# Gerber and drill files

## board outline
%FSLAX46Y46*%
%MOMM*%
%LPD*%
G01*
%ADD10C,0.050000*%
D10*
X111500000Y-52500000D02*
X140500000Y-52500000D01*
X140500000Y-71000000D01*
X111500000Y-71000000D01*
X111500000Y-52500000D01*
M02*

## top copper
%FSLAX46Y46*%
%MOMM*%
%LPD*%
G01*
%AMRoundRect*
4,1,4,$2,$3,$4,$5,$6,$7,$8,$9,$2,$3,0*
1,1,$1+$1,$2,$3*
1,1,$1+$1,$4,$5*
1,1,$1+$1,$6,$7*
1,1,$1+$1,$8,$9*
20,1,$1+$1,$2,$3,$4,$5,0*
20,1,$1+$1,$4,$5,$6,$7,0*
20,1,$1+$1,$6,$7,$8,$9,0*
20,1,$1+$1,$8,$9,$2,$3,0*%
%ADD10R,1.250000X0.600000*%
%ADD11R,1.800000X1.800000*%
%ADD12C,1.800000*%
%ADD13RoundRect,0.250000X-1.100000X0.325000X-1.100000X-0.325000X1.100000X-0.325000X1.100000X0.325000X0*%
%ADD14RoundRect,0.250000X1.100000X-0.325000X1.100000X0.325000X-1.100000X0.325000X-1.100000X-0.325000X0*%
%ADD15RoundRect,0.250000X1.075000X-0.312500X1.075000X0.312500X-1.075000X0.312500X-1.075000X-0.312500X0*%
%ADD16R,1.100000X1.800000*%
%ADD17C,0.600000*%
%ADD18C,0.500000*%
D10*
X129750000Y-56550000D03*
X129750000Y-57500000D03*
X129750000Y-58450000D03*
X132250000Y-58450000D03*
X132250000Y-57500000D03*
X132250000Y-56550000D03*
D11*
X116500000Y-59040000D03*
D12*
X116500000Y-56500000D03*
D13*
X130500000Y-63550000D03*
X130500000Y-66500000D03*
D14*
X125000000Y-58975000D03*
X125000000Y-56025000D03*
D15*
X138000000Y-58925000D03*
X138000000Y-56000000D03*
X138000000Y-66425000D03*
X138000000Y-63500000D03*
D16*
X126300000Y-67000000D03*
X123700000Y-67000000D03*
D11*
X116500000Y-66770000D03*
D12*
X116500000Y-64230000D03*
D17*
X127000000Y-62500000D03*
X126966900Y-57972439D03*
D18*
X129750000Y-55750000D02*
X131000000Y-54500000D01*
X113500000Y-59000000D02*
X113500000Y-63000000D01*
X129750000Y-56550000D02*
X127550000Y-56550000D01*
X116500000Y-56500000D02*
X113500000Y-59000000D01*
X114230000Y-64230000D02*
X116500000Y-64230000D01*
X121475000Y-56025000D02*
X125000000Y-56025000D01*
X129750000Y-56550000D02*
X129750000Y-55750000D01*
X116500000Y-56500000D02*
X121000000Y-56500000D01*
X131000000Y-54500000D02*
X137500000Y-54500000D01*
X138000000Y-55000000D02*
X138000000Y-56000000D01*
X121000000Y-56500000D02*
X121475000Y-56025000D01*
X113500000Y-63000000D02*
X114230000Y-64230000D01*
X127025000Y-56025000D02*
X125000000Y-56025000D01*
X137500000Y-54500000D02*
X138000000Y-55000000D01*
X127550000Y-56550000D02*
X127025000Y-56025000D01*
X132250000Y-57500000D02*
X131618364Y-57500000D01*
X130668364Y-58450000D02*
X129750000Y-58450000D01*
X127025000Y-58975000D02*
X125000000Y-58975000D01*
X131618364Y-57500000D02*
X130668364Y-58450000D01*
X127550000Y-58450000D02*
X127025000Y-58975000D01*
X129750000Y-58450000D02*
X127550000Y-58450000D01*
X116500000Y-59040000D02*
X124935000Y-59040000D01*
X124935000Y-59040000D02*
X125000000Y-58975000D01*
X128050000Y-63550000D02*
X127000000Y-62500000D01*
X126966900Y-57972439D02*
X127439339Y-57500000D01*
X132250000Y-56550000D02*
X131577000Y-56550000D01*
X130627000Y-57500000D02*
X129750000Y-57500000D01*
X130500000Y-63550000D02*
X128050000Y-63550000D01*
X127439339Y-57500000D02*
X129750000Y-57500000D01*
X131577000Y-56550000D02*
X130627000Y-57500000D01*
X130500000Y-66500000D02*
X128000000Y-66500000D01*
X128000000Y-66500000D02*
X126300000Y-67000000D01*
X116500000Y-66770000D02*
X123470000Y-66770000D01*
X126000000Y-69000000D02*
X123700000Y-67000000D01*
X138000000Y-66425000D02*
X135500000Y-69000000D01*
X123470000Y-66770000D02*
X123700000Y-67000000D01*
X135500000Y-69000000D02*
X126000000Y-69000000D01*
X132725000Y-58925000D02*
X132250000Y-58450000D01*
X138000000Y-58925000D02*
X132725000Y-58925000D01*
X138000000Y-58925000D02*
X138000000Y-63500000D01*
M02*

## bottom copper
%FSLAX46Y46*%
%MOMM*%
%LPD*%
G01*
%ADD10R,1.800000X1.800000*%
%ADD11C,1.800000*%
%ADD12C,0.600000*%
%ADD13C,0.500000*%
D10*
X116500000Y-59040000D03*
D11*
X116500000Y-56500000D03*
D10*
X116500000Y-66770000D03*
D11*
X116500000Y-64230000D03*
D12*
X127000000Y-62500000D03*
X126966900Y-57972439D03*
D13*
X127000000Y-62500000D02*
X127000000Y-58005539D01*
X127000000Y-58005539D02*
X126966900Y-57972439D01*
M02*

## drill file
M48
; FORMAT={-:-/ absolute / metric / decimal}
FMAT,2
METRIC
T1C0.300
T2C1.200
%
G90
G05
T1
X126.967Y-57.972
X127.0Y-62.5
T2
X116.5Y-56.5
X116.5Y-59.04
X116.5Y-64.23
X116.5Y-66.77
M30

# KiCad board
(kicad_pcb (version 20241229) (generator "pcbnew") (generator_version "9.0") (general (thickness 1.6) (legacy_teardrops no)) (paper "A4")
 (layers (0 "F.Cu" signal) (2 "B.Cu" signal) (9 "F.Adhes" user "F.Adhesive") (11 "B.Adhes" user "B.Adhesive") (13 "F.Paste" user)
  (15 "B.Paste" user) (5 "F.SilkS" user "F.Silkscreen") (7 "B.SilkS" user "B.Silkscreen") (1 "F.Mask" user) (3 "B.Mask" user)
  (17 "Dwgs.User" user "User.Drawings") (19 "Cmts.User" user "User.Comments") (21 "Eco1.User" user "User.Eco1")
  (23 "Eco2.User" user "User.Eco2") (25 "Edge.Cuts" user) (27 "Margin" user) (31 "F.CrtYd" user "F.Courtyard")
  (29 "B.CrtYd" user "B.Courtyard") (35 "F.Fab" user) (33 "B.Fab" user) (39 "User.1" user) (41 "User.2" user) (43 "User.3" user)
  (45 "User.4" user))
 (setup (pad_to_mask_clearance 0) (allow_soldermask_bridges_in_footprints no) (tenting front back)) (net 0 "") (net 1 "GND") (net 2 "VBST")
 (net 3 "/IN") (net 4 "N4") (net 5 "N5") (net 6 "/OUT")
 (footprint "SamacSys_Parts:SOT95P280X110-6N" (layer "F.Cu") (at 131 57.5)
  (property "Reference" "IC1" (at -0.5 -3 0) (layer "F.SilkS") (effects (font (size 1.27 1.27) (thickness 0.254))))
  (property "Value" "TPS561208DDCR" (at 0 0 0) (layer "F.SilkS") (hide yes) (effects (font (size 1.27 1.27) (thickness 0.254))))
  (pad "1" smd rect (at -1.25 -0.95 90) (size 0.6 1.25) (layers "F.Cu" "F.Mask" "F.Paste") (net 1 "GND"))
  (pad "2" smd rect (at -1.25 0 90) (size 0.6 1.25) (layers "F.Cu" "F.Mask" "F.Paste") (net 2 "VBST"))
  (pad "3" smd rect (at -1.25 0.95 90) (size 0.6 1.25) (layers "F.Cu" "F.Mask" "F.Paste") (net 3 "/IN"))
  (pad "4" smd rect (at 1.25 0.95 90) (size 0.6 1.25) (layers "F.Cu" "F.Mask" "F.Paste") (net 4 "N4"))
  (pad "5" smd rect (at 1.25 0 90) (size 0.6 1.25) (layers "F.Cu" "F.Mask" "F.Paste") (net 3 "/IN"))
  (pad "6" smd rect (at 1.25 -0.95 90) (size 0.6 1.25) (layers "F.Cu" "F.Mask" "F.Paste") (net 2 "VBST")))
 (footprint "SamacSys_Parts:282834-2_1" (layer "F.Cu") (at 116.5 59.04 90)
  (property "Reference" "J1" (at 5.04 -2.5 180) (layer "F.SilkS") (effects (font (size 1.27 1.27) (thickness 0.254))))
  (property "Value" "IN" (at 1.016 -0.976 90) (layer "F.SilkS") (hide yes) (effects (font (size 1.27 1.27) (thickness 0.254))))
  (pad "1" thru_hole rect (at 0 0 90) (size 1.8 1.8) (drill 1.2) (layers "*.Cu" "*.Mask") (remove_unused_layers no) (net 3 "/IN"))
  (pad "2" thru_hole circle (at 2.54 0 90) (size 1.8 1.8) (drill 1.2) (layers "*.Cu" "*.Mask") (remove_unused_layers no) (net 1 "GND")))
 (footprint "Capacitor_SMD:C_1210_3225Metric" (layer "F.Cu") (at 130.5 65.025 -90)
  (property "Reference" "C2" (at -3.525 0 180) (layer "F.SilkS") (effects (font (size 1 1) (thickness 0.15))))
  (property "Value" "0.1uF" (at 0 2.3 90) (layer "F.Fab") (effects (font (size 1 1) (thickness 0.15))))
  (pad "1" smd roundrect (at -1.475 0 270) (size 1.15 2.7) (layers "F.Cu" "F.Mask" "F.Paste") (roundrect_rratio 0.217391) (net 2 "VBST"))
  (pad "2" smd roundrect (at 1.475 0 270) (size 1.15 2.7) (layers "F.Cu" "F.Mask" "F.Paste") (roundrect_rratio 0.217391) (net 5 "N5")))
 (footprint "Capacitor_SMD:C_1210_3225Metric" (layer "F.Cu") (at 125 57.5 90)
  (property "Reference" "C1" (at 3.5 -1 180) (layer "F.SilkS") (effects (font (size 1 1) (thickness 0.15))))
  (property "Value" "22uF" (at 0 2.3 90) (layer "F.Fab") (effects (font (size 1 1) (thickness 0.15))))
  (pad "1" smd roundrect (at -1.475 0 90) (size 1.15 2.7) (layers "F.Cu" "F.Mask" "F.Paste") (roundrect_rratio 0.217391) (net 3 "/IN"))
  (pad "2" smd roundrect (at 1.475 0 90) (size 1.15 2.7) (layers "F.Cu" "F.Mask" "F.Paste") (roundrect_rratio 0.217391) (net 1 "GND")))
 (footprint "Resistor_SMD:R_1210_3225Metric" (layer "F.Cu") (at 138 57.4625 90)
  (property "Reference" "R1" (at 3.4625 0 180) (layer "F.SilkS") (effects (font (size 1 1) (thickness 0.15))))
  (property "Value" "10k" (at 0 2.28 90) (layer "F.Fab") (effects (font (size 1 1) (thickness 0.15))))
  (pad "1" smd roundrect (at -1.4625 0 90) (size 1.125 2.65) (layers "F.Cu" "F.Mask" "F.Paste") (roundrect_rratio 0.222222) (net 4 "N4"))
  (pad "2" smd roundrect (at 1.4625 0 90) (size 1.125 2.65) (layers "F.Cu" "F.Mask" "F.Paste") (roundrect_rratio 0.222222) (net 1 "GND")))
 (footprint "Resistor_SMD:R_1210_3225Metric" (layer "F.Cu") (at 138 64.9625 90)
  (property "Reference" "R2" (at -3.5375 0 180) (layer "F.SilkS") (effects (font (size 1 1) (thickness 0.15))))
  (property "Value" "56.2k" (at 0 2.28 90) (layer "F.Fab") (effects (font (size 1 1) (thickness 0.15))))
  (pad "1" smd roundrect (at -1.4625 0 90) (size 1.125 2.65) (layers "F.Cu" "F.Mask" "F.Paste") (roundrect_rratio 0.222222) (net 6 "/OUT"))
  (pad "2" smd roundrect (at 1.4625 0 90) (size 1.125 2.65) (layers "F.Cu" "F.Mask" "F.Paste") (roundrect_rratio 0.222222) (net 4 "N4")))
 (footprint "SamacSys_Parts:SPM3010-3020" (layer "F.Cu") (at 125 67 180)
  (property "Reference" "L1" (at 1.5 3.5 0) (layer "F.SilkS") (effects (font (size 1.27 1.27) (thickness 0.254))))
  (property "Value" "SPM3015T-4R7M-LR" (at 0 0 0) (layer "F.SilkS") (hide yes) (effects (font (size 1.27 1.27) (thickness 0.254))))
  (pad "1" smd rect (at -1.3 0 180) (size 1.1 1.8) (layers "F.Cu" "F.Mask" "F.Paste") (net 5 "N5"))
  (pad "2" smd rect (at 1.3 0 180) (size 1.1 1.8) (layers "F.Cu" "F.Mask" "F.Paste") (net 6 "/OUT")))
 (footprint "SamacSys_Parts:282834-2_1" (layer "F.Cu") (at 116.5 66.77 90)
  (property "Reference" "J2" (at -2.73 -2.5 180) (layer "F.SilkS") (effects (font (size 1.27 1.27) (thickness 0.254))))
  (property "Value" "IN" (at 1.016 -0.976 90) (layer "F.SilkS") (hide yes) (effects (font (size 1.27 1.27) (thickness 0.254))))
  (pad "1" thru_hole rect (at 0 0 90) (size 1.8 1.8) (drill 1.2) (layers "*.Cu" "*.Mask") (remove_unused_layers no) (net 6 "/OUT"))
  (pad "2" thru_hole circle (at 2.54 0 90) (size 1.8 1.8) (drill 1.2) (layers "*.Cu" "*.Mask") (remove_unused_layers no) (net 1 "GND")))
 (gr_rect (start 111.5 52.5) (end 140.5 71) (stroke (width 0.05) (type default)) (fill no) (layer "Edge.Cuts"))
 (segment (start 129.75 55.75) (end 131 54.5) (width 0.5) (layer "F.Cu") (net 1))
 (segment (start 113.5 59) (end 113.5 63) (width 0.5) (layer "F.Cu") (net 1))
 (segment (start 129.75 56.55) (end 127.55 56.55) (width 0.5) (layer "F.Cu") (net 1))
 (segment (start 116.5 56.5) (end 113.5 59) (width 0.5) (layer "F.Cu") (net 1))
 (segment (start 114.23 64.23) (end 116.5 64.23) (width 0.5) (layer "F.Cu") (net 1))
 (segment (start 121.475 56.025) (end 125 56.025) (width 0.5) (layer "F.Cu") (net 1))
 (segment (start 129.75 56.55) (end 129.75 55.75) (width 0.5) (layer "F.Cu") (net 1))
 (segment (start 116.5 56.5) (end 121 56.5) (width 0.5) (layer "F.Cu") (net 1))
 (segment (start 131 54.5) (end 137.5 54.5) (width 0.5) (layer "F.Cu") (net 1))
 (segment (start 138 55) (end 138 56) (width 0.5) (layer "F.Cu") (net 1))
 (segment (start 121 56.5) (end 121.475 56.025) (width 0.5) (layer "F.Cu") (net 1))
 (segment (start 113.5 63) (end 114.23 64.23) (width 0.5) (layer "F.Cu") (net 1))
 (segment (start 127.025 56.025) (end 125 56.025) (width 0.5) (layer "F.Cu") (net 1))
 (segment (start 137.5 54.5) (end 138 55) (width 0.5) (layer "F.Cu") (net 1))
 (segment (start 127.55 56.55) (end 127.025 56.025) (width 0.5) (layer "F.Cu") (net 1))
 (segment (start 132.25 57.5) (end 131.618364 57.5) (width 0.5) (layer "F.Cu") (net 3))
 (segment (start 130.668364 58.45) (end 129.75 58.45) (width 0.5) (layer "F.Cu") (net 3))
 (segment (start 127.025 58.975) (end 125 58.975) (width 0.5) (layer "F.Cu") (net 3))
 (segment (start 131.618364 57.5) (end 130.668364 58.45) (width 0.5) (layer "F.Cu") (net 3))
 (segment (start 127.55 58.45) (end 127.025 58.975) (width 0.5) (layer "F.Cu") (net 3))
 (segment (start 129.75 58.45) (end 127.55 58.45) (width 0.5) (layer "F.Cu") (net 3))
 (segment (start 116.5 59.04) (end 124.935 59.04) (width 0.5) (layer "F.Cu") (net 3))
 (segment (start 124.935 59.04) (end 125 58.975) (width 0.5) (layer "F.Cu") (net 3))
 (segment (start 128.05 63.55) (end 127 62.5) (width 0.5) (layer "F.Cu") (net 2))
 (segment (start 126.9669 57.972439) (end 127.439339 57.5) (width 0.5) (layer "F.Cu") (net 2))
 (segment (start 132.25 56.55) (end 131.577 56.55) (width 0.5) (layer "F.Cu") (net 2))
 (segment (start 130.627 57.5) (end 129.75 57.5) (width 0.5) (layer "F.Cu") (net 2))
 (segment (start 130.5 63.55) (end 128.05 63.55) (width 0.5) (layer "F.Cu") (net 2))
 (segment (start 127.439339 57.5) (end 129.75 57.5) (width 0.5) (layer "F.Cu") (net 2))
 (segment (start 131.577 56.55) (end 130.627 57.5) (width 0.5) (layer "F.Cu") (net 2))
 (via (at 127 62.5) (size 0.6) (drill 0.3) (layers "F.Cu" "B.Cu") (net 2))
 (via (at 126.9669 57.972439) (size 0.6) (drill 0.3) (layers "F.Cu" "B.Cu") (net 2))
 (segment (start 127 62.5) (end 127 58.005539) (width 0.5) (layer "B.Cu") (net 2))
 (segment (start 127 58.005539) (end 126.9669 57.972439) (width 0.5) (layer "B.Cu") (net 2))
 (segment (start 130.5 66.5) (end 128 66.5) (width 0.5) (layer "F.Cu") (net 5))
 (segment (start 128 66.5) (end 126.3 67) (width 0.5) (layer "F.Cu") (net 5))
 (segment (start 116.5 66.77) (end 123.47 66.77) (width 0.5) (layer "F.Cu") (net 6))
 (segment (start 126 69) (end 123.7 67) (width 0.5) (layer "F.Cu") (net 6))
 (segment (start 138 66.425) (end 135.5 69) (width 0.5) (layer "F.Cu") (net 6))
 (segment (start 123.47 66.77) (end 123.7 67) (width 0.5) (layer "F.Cu") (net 6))
 (segment (start 135.5 69) (end 126 69) (width 0.5) (layer "F.Cu") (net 6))
 (segment (start 132.725 58.925) (end 132.25 58.45) (width 0.5) (layer "F.Cu") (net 4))
 (segment (start 138 58.925) (end 132.725 58.925) (width 0.5) (layer "F.Cu") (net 4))
 (segment (start 138 58.925) (end 138 63.5) (width 0.5) (layer "F.Cu") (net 4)))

